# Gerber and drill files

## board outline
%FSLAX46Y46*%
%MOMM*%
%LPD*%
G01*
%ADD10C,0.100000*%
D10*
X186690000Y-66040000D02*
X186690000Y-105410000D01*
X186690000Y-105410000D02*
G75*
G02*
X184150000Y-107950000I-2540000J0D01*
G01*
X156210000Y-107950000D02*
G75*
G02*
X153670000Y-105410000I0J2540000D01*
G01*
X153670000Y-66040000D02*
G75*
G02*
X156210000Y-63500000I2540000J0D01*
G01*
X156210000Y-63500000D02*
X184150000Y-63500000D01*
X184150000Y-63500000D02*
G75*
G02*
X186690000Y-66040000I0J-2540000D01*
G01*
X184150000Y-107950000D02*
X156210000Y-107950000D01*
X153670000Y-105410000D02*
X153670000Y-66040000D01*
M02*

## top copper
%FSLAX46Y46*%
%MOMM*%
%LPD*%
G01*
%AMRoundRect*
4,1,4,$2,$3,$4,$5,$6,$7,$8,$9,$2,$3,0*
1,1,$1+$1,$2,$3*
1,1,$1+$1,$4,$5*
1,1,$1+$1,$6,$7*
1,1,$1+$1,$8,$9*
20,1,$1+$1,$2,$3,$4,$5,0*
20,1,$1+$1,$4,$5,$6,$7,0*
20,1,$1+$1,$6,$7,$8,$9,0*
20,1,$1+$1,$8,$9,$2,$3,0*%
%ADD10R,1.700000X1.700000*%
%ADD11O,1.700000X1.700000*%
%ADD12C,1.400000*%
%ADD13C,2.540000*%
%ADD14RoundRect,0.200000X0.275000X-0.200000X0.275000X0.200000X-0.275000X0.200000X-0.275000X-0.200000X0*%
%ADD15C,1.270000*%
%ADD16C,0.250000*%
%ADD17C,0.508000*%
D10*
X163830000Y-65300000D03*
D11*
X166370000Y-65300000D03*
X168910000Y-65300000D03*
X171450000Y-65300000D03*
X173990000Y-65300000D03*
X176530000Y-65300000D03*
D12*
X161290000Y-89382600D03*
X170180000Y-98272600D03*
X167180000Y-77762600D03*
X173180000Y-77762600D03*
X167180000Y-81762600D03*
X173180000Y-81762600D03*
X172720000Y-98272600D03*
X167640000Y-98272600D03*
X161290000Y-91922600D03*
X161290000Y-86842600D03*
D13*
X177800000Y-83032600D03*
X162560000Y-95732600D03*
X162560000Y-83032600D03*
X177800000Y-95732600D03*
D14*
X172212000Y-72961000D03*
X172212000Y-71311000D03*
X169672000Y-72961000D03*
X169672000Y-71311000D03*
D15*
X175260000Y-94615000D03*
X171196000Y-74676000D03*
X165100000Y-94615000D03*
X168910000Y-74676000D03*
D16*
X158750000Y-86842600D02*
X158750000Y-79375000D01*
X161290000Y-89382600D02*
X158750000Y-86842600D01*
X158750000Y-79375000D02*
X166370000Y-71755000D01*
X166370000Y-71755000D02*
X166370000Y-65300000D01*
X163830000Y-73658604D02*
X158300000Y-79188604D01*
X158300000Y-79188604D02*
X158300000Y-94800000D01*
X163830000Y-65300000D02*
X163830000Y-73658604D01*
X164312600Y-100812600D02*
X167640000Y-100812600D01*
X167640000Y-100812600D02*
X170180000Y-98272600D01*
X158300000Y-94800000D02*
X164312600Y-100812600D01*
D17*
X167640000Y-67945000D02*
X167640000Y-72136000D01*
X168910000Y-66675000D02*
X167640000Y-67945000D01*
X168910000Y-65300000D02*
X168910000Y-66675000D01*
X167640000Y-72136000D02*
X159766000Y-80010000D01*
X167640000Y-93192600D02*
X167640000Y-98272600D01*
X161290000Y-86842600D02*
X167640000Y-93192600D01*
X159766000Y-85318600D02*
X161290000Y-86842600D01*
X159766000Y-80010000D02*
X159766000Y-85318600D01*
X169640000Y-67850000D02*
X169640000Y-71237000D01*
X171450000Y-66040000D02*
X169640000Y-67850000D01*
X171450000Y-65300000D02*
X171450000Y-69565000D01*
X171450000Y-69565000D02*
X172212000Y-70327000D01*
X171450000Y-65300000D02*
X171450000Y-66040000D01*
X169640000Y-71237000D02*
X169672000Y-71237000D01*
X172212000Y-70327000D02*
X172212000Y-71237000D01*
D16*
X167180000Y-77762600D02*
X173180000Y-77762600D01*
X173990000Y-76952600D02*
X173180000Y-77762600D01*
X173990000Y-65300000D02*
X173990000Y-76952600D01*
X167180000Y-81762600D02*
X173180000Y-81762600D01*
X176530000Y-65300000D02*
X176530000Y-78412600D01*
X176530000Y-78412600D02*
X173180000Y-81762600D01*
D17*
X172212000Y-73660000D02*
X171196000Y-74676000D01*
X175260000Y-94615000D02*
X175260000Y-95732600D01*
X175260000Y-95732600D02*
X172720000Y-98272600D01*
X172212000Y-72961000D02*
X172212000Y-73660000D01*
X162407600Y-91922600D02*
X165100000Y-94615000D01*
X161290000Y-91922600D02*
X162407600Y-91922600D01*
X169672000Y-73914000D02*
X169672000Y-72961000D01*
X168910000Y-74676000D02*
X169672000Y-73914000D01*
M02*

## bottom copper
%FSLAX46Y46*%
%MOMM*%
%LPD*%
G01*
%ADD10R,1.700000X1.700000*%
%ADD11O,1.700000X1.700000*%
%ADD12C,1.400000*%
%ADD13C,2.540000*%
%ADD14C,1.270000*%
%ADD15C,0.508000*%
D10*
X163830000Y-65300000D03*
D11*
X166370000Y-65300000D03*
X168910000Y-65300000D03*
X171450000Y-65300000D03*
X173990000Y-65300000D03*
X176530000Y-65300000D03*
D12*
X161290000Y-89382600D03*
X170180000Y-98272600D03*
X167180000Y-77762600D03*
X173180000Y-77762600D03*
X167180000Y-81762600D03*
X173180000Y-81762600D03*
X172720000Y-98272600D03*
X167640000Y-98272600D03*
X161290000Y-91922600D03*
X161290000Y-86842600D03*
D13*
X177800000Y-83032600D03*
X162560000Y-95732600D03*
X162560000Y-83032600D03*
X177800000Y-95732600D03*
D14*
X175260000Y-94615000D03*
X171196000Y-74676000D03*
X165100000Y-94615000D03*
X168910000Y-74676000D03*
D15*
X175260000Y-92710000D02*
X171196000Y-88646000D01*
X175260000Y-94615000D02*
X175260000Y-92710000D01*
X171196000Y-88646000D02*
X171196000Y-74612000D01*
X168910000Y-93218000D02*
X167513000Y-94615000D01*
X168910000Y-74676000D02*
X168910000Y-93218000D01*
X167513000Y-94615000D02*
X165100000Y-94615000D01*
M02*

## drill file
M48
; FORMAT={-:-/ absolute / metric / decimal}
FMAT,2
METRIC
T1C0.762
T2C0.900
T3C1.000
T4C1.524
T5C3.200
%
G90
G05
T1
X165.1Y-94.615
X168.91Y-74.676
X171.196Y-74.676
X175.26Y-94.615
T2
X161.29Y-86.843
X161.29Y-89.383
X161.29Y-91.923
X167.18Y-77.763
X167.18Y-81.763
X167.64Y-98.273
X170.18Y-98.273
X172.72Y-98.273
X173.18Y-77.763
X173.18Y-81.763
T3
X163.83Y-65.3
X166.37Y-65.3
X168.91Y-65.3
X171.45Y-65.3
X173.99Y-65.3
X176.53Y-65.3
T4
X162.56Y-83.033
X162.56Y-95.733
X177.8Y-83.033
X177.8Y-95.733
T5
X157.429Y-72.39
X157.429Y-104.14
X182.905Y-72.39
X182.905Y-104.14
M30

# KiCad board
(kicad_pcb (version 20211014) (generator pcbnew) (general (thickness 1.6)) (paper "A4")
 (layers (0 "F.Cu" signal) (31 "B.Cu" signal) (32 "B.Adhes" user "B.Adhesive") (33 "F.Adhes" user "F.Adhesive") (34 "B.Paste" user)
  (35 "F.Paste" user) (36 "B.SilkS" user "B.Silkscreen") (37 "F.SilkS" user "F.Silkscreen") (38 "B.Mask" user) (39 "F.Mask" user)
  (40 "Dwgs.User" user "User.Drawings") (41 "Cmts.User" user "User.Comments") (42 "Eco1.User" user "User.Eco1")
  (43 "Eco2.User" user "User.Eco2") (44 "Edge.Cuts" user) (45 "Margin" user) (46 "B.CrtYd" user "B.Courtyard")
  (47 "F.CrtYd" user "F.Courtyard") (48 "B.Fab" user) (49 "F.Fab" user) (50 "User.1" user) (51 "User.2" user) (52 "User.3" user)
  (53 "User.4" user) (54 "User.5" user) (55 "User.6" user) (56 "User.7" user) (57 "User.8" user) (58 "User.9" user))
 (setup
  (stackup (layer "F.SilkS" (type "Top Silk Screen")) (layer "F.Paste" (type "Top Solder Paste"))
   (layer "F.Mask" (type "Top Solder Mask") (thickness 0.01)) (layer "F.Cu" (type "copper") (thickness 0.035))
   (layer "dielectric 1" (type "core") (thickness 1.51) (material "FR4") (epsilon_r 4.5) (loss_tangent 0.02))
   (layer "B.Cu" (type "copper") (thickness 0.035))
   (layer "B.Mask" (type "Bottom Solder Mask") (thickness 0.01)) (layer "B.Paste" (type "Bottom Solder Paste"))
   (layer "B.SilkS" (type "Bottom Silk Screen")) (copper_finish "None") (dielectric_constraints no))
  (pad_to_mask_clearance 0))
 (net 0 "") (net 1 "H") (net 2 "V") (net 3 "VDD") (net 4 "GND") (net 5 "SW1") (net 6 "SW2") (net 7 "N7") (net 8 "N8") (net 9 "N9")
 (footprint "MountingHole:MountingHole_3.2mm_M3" (layer "F.Cu") (at 182.9054 104.14)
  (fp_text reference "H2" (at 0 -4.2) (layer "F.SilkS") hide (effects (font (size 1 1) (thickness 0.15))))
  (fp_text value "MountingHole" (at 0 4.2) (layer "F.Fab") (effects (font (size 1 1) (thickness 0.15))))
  (pad "" np_thru_hole circle (at 0 0) (size 3.2 3.2) (drill 3.2) (layers *.Cu *.Mask)))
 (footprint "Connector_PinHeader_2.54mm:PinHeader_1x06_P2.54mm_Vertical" (layer "F.Cu") (at 163.83 65.3 90)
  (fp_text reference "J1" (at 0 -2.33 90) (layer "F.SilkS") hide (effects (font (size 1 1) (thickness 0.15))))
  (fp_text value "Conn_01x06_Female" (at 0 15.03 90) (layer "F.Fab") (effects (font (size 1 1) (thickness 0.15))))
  (pad "1" thru_hole rect (at 0 0 90) (size 1.7 1.7) (drill 1) (layers *.Cu *.Mask) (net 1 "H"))
  (pad "2" thru_hole oval (at 0 2.54 90) (size 1.7 1.7) (drill 1) (layers *.Cu *.Mask) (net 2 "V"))
  (pad "3" thru_hole oval (at 0 5.08 90) (size 1.7 1.7) (drill 1) (layers *.Cu *.Mask) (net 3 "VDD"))
  (pad "4" thru_hole oval (at 0 7.62 90) (size 1.7 1.7) (drill 1) (layers *.Cu *.Mask) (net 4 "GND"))
  (pad "5" thru_hole oval (at 0 10.16 90) (size 1.7 1.7) (drill 1) (layers *.Cu *.Mask) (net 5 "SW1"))
  (pad "6" thru_hole oval (at 0 12.7 90) (size 1.7 1.7) (drill 1) (layers *.Cu *.Mask) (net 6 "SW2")))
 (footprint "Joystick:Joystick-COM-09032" (layer "F.Cu") (at 170.18 89.3826)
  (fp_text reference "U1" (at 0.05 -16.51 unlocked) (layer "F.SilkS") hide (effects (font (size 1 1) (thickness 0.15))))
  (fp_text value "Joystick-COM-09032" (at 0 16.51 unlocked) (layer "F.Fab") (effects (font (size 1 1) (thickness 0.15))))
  (pad "1" thru_hole circle (at -8.89 0 90) (size 1.4 1.4) (drill 0.9) (layers *.Cu *.Mask) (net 2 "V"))
  (pad "2" thru_hole circle (at 0 8.89) (size 1.4 1.4) (drill 0.9) (layers *.Cu *.Mask) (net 1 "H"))
  (pad "3" thru_hole circle (at -3 -11.62) (size 1.4 1.4) (drill 0.9) (layers *.Cu *.Mask) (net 5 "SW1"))
  (pad "3" thru_hole circle (at 3 -11.62) (size 1.4 1.4) (drill 0.9) (layers *.Cu *.Mask) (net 5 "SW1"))
  (pad "4" thru_hole circle (at -3 -7.62) (size 1.4 1.4) (drill 0.9) (layers *.Cu *.Mask) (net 6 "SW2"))
  (pad "4" thru_hole circle (at 3 -7.62) (size 1.4 1.4) (drill 0.9) (layers *.Cu *.Mask) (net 6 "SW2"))
  (pad "5" thru_hole circle (at 2.54 8.89) (size 1.4 1.4) (drill 0.9) (layers *.Cu *.Mask) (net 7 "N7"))
  (pad "6" thru_hole circle (at -2.54 8.89) (size 1.4 1.4) (drill 0.9) (layers *.Cu *.Mask) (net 3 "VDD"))
  (pad "7" thru_hole circle (at -8.89 2.54 90) (size 1.4 1.4) (drill 0.9) (layers *.Cu *.Mask) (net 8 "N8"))
  (pad "8" thru_hole circle (at -8.89 -2.54 90) (size 1.4 1.4) (drill 0.9) (layers *.Cu *.Mask) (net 3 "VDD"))
  (pad "9" thru_hole circle (at 7.62 -6.35) (size 2.54 2.54) (drill 1.524) (layers *.Cu *.Mask) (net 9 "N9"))
  (pad "9" thru_hole circle (at -7.62 6.35) (size 2.54 2.54) (drill 1.524) (layers *.Cu *.Mask) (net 9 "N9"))
  (pad "9" thru_hole circle (at -7.62 -6.35) (size 2.54 2.54) (drill 1.524) (layers *.Cu *.Mask) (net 9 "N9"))
  (pad "9" thru_hole circle (at 7.62 6.35) (size 2.54 2.54) (drill 1.524) (layers *.Cu *.Mask) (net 9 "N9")))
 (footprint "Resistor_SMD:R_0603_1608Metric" (layer "F.Cu") (at 172.212 72.136 90)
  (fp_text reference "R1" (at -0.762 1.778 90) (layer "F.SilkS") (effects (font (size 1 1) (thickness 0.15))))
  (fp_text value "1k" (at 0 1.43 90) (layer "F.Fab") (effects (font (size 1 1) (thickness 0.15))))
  (pad "1" smd roundrect (at -0.825 0 90) (size 0.8 0.95) (layers "F.Cu" "F.Paste" "F.Mask") (roundrect_rratio 0.25) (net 7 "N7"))
  (pad "2" smd roundrect (at 0.825 0 90) (size 0.8 0.95) (layers "F.Cu" "F.Paste" "F.Mask") (roundrect_rratio 0.25) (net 4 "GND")))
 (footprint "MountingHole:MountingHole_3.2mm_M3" (layer "F.Cu") (at 157.4292 72.39)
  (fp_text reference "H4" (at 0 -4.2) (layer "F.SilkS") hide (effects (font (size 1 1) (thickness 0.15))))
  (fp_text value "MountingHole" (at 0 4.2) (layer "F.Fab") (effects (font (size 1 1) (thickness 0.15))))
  (pad "" np_thru_hole circle (at 0 0) (size 3.2 3.2) (drill 3.2) (layers *.Cu *.Mask)))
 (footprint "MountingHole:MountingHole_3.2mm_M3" (layer "F.Cu") (at 182.9054 72.39)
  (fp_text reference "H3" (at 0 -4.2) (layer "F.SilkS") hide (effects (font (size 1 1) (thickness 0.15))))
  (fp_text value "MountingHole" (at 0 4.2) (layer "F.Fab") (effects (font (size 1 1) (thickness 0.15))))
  (pad "" np_thru_hole circle (at 0 0) (size 3.2 3.2) (drill 3.2) (layers *.Cu *.Mask)))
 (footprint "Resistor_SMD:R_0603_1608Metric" (layer "F.Cu") (at 169.672 72.136 90)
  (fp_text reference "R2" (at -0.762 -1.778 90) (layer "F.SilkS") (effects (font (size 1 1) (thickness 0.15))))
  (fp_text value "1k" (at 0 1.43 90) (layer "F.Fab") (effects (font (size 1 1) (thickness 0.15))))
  (pad "1" smd roundrect (at -0.825 0 90) (size 0.8 0.95) (layers "F.Cu" "F.Paste" "F.Mask") (roundrect_rratio 0.25) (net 8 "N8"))
  (pad "2" smd roundrect (at 0.825 0 90) (size 0.8 0.95) (layers "F.Cu" "F.Paste" "F.Mask") (roundrect_rratio 0.25) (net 4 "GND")))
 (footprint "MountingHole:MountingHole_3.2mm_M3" (layer "F.Cu") (at 157.4292 104.14)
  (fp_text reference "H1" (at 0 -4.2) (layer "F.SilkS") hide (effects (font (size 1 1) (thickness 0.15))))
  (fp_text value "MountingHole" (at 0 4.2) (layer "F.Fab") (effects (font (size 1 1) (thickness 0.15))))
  (pad "" np_thru_hole circle (at 0 0) (size 3.2 3.2) (drill 3.2) (layers *.Cu *.Mask)))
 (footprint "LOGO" (layer "B.Cu") (at 170.6 89.5 -90)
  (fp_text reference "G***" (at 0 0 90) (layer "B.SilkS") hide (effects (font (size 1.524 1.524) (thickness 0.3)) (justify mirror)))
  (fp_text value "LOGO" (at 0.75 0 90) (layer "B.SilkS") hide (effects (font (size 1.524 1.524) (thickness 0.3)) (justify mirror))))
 (gr_line (start 186.69 66.04) (end 186.69 105.41) (layer "Edge.Cuts") (width 0.1))
 (gr_arc (start 186.69 105.41) (mid 185.946051 107.206051) (end 184.15 107.95) (layer "Edge.Cuts") (width 0.1))
 (gr_arc (start 156.21 107.95) (mid 154.413949 107.206051) (end 153.67 105.41) (layer "Edge.Cuts") (width 0.1))
 (gr_arc (start 153.67 66.04) (mid 154.413949 64.243949) (end 156.21 63.5) (layer "Edge.Cuts") (width 0.1))
 (gr_line (start 156.21 63.5) (end 184.15 63.5) (layer "Edge.Cuts") (width 0.1))
 (gr_arc (start 184.15 63.5) (mid 185.946051 64.243949) (end 186.69 66.04) (layer "Edge.Cuts") (width 0.1))
 (gr_line (start 184.15 107.95) (end 156.21 107.95) (layer "Edge.Cuts") (width 0.1))
 (gr_line (start 153.67 105.41) (end 153.67 66.04) (layer "Edge.Cuts") (width 0.1))
 (segment (start 158.75 86.8426) (end 158.75 79.375) (width 0.25) (layer "F.Cu") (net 2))
 (segment (start 161.29 89.3826) (end 158.75 86.8426) (width 0.25) (layer "F.Cu") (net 2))
 (segment (start 158.75 79.375) (end 166.37 71.755) (width 0.25) (layer "F.Cu") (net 2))
 (segment (start 166.37 71.755) (end 166.37 65.3) (width 0.25) (layer "F.Cu") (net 2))
 (segment (start 163.83 73.658604) (end 158.3 79.188604) (width 0.25) (layer "F.Cu") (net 1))
 (segment (start 158.3 79.188604) (end 158.3 94.8) (width 0.25) (layer "F.Cu") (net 1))
 (segment (start 163.83 65.3) (end 163.83 73.658604) (width 0.25) (layer "F.Cu") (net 1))
 (segment (start 164.3126 100.8126) (end 167.64 100.8126) (width 0.25) (layer "F.Cu") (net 1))
 (segment (start 167.64 100.8126) (end 170.18 98.2726) (width 0.25) (layer "F.Cu") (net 1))
 (segment (start 158.3 94.8) (end 164.3126 100.8126) (width 0.25) (layer "F.Cu") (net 1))
 (segment (start 167.64 67.945) (end 167.64 72.136) (width 0.508) (layer "F.Cu") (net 3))
 (segment (start 168.91 66.675) (end 167.64 67.945) (width 0.508) (layer "F.Cu") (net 3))
 (segment (start 168.91 65.3) (end 168.91 66.675) (width 0.508) (layer "F.Cu") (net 3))
 (segment (start 167.64 72.136) (end 159.766 80.01) (width 0.508) (layer "F.Cu") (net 3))
 (segment (start 167.64 93.1926) (end 167.64 98.2726) (width 0.508) (layer "F.Cu") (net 3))
 (segment (start 161.29 86.8426) (end 167.64 93.1926) (width 0.508) (layer "F.Cu") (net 3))
 (segment (start 159.766 85.3186) (end 161.29 86.8426) (width 0.508) (layer "F.Cu") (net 3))
 (segment (start 159.766 80.01) (end 159.766 85.3186) (width 0.508) (layer "F.Cu") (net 3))
 (segment (start 169.64 67.85) (end 169.64 71.237) (width 0.508) (layer "F.Cu") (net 4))
 (segment (start 171.45 66.04) (end 169.64 67.85) (width 0.508) (layer "F.Cu") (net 4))
 (segment (start 171.45 65.3) (end 171.45 69.565) (width 0.508) (layer "F.Cu") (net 4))
 (segment (start 171.45 69.565) (end 172.212 70.327) (width 0.508) (layer "F.Cu") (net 4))
 (segment (start 171.45 65.3) (end 171.45 66.04) (width 0.508) (layer "F.Cu") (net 4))
 (segment (start 169.64 71.237) (end 169.672 71.237) (width 0.508) (layer "F.Cu") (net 4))
 (segment (start 172.212 70.327) (end 172.212 71.237) (width 0.508) (layer "F.Cu") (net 4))
 (segment (start 167.18 77.7626) (end 173.18 77.7626) (width 0.25) (layer "F.Cu") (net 5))
 (segment (start 173.99 76.9526) (end 173.18 77.7626) (width 0.25) (layer "F.Cu") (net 5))
 (segment (start 173.99 65.3) (end 173.99 76.9526) (width 0.25) (layer "F.Cu") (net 5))
 (segment (start 167.18 81.7626) (end 173.18 81.7626) (width 0.25) (layer "F.Cu") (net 6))
 (segment (start 176.53 65.3) (end 176.53 78.4126) (width 0.25) (layer "F.Cu") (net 6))
 (segment (start 176.53 78.4126) (end 173.18 81.7626) (width 0.25) (layer "F.Cu") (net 6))
 (segment (start 172.212 73.66) (end 171.196 74.676) (width 0.508) (layer "F.Cu") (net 7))
 (segment (start 175.26 94.615) (end 175.26 95.7326) (width 0.508) (layer "F.Cu") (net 7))
 (segment (start 175.26 95.7326) (end 172.72 98.2726) (width 0.508) (layer "F.Cu") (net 7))
 (segment (start 172.212 72.961) (end 172.212 73.66) (width 0.508) (layer "F.Cu") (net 7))
 (via (at 175.26 94.615) (size 1.27) (drill 0.762) (layers "F.Cu" "B.Cu") (free) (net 7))
 (via (at 171.196 74.676) (size 1.27) (drill 0.762) (layers "F.Cu" "B.Cu") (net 7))
 (segment (start 175.26 92.71) (end 171.196 88.646) (width 0.508) (layer "B.Cu") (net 7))
 (segment (start 175.26 94.615) (end 175.26 92.71) (width 0.508) (layer "B.Cu") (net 7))
 (segment (start 171.196 88.646) (end 171.196 74.612) (width 0.508) (layer "B.Cu") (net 7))
 (segment (start 162.4076 91.9226) (end 165.1 94.615) (width 0.508) (layer "F.Cu") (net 8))
 (segment (start 161.29 91.9226) (end 162.4076 91.9226) (width 0.508) (layer "F.Cu") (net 8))
 (segment (start 169.672 73.914) (end 169.672 72.961) (width 0.508) (layer "F.Cu") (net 8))
 (segment (start 168.91 74.676) (end 169.672 73.914) (width 0.508) (layer "F.Cu") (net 8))
 (via (at 165.1 94.615) (size 1.27) (drill 0.762) (layers "F.Cu" "B.Cu") (free) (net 8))
 (via (at 168.91 74.676) (size 1.27) (drill 0.762) (layers "F.Cu" "B.Cu") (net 8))
 (segment (start 168.91 93.218) (end 167.513 94.615) (width 0.508) (layer "B.Cu") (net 8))
 (segment (start 168.91 74.676) (end 168.91 93.218) (width 0.508) (layer "B.Cu") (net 8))
 (segment (start 167.513 94.615) (end 165.1 94.615) (width 0.508) (layer "B.Cu") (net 8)))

